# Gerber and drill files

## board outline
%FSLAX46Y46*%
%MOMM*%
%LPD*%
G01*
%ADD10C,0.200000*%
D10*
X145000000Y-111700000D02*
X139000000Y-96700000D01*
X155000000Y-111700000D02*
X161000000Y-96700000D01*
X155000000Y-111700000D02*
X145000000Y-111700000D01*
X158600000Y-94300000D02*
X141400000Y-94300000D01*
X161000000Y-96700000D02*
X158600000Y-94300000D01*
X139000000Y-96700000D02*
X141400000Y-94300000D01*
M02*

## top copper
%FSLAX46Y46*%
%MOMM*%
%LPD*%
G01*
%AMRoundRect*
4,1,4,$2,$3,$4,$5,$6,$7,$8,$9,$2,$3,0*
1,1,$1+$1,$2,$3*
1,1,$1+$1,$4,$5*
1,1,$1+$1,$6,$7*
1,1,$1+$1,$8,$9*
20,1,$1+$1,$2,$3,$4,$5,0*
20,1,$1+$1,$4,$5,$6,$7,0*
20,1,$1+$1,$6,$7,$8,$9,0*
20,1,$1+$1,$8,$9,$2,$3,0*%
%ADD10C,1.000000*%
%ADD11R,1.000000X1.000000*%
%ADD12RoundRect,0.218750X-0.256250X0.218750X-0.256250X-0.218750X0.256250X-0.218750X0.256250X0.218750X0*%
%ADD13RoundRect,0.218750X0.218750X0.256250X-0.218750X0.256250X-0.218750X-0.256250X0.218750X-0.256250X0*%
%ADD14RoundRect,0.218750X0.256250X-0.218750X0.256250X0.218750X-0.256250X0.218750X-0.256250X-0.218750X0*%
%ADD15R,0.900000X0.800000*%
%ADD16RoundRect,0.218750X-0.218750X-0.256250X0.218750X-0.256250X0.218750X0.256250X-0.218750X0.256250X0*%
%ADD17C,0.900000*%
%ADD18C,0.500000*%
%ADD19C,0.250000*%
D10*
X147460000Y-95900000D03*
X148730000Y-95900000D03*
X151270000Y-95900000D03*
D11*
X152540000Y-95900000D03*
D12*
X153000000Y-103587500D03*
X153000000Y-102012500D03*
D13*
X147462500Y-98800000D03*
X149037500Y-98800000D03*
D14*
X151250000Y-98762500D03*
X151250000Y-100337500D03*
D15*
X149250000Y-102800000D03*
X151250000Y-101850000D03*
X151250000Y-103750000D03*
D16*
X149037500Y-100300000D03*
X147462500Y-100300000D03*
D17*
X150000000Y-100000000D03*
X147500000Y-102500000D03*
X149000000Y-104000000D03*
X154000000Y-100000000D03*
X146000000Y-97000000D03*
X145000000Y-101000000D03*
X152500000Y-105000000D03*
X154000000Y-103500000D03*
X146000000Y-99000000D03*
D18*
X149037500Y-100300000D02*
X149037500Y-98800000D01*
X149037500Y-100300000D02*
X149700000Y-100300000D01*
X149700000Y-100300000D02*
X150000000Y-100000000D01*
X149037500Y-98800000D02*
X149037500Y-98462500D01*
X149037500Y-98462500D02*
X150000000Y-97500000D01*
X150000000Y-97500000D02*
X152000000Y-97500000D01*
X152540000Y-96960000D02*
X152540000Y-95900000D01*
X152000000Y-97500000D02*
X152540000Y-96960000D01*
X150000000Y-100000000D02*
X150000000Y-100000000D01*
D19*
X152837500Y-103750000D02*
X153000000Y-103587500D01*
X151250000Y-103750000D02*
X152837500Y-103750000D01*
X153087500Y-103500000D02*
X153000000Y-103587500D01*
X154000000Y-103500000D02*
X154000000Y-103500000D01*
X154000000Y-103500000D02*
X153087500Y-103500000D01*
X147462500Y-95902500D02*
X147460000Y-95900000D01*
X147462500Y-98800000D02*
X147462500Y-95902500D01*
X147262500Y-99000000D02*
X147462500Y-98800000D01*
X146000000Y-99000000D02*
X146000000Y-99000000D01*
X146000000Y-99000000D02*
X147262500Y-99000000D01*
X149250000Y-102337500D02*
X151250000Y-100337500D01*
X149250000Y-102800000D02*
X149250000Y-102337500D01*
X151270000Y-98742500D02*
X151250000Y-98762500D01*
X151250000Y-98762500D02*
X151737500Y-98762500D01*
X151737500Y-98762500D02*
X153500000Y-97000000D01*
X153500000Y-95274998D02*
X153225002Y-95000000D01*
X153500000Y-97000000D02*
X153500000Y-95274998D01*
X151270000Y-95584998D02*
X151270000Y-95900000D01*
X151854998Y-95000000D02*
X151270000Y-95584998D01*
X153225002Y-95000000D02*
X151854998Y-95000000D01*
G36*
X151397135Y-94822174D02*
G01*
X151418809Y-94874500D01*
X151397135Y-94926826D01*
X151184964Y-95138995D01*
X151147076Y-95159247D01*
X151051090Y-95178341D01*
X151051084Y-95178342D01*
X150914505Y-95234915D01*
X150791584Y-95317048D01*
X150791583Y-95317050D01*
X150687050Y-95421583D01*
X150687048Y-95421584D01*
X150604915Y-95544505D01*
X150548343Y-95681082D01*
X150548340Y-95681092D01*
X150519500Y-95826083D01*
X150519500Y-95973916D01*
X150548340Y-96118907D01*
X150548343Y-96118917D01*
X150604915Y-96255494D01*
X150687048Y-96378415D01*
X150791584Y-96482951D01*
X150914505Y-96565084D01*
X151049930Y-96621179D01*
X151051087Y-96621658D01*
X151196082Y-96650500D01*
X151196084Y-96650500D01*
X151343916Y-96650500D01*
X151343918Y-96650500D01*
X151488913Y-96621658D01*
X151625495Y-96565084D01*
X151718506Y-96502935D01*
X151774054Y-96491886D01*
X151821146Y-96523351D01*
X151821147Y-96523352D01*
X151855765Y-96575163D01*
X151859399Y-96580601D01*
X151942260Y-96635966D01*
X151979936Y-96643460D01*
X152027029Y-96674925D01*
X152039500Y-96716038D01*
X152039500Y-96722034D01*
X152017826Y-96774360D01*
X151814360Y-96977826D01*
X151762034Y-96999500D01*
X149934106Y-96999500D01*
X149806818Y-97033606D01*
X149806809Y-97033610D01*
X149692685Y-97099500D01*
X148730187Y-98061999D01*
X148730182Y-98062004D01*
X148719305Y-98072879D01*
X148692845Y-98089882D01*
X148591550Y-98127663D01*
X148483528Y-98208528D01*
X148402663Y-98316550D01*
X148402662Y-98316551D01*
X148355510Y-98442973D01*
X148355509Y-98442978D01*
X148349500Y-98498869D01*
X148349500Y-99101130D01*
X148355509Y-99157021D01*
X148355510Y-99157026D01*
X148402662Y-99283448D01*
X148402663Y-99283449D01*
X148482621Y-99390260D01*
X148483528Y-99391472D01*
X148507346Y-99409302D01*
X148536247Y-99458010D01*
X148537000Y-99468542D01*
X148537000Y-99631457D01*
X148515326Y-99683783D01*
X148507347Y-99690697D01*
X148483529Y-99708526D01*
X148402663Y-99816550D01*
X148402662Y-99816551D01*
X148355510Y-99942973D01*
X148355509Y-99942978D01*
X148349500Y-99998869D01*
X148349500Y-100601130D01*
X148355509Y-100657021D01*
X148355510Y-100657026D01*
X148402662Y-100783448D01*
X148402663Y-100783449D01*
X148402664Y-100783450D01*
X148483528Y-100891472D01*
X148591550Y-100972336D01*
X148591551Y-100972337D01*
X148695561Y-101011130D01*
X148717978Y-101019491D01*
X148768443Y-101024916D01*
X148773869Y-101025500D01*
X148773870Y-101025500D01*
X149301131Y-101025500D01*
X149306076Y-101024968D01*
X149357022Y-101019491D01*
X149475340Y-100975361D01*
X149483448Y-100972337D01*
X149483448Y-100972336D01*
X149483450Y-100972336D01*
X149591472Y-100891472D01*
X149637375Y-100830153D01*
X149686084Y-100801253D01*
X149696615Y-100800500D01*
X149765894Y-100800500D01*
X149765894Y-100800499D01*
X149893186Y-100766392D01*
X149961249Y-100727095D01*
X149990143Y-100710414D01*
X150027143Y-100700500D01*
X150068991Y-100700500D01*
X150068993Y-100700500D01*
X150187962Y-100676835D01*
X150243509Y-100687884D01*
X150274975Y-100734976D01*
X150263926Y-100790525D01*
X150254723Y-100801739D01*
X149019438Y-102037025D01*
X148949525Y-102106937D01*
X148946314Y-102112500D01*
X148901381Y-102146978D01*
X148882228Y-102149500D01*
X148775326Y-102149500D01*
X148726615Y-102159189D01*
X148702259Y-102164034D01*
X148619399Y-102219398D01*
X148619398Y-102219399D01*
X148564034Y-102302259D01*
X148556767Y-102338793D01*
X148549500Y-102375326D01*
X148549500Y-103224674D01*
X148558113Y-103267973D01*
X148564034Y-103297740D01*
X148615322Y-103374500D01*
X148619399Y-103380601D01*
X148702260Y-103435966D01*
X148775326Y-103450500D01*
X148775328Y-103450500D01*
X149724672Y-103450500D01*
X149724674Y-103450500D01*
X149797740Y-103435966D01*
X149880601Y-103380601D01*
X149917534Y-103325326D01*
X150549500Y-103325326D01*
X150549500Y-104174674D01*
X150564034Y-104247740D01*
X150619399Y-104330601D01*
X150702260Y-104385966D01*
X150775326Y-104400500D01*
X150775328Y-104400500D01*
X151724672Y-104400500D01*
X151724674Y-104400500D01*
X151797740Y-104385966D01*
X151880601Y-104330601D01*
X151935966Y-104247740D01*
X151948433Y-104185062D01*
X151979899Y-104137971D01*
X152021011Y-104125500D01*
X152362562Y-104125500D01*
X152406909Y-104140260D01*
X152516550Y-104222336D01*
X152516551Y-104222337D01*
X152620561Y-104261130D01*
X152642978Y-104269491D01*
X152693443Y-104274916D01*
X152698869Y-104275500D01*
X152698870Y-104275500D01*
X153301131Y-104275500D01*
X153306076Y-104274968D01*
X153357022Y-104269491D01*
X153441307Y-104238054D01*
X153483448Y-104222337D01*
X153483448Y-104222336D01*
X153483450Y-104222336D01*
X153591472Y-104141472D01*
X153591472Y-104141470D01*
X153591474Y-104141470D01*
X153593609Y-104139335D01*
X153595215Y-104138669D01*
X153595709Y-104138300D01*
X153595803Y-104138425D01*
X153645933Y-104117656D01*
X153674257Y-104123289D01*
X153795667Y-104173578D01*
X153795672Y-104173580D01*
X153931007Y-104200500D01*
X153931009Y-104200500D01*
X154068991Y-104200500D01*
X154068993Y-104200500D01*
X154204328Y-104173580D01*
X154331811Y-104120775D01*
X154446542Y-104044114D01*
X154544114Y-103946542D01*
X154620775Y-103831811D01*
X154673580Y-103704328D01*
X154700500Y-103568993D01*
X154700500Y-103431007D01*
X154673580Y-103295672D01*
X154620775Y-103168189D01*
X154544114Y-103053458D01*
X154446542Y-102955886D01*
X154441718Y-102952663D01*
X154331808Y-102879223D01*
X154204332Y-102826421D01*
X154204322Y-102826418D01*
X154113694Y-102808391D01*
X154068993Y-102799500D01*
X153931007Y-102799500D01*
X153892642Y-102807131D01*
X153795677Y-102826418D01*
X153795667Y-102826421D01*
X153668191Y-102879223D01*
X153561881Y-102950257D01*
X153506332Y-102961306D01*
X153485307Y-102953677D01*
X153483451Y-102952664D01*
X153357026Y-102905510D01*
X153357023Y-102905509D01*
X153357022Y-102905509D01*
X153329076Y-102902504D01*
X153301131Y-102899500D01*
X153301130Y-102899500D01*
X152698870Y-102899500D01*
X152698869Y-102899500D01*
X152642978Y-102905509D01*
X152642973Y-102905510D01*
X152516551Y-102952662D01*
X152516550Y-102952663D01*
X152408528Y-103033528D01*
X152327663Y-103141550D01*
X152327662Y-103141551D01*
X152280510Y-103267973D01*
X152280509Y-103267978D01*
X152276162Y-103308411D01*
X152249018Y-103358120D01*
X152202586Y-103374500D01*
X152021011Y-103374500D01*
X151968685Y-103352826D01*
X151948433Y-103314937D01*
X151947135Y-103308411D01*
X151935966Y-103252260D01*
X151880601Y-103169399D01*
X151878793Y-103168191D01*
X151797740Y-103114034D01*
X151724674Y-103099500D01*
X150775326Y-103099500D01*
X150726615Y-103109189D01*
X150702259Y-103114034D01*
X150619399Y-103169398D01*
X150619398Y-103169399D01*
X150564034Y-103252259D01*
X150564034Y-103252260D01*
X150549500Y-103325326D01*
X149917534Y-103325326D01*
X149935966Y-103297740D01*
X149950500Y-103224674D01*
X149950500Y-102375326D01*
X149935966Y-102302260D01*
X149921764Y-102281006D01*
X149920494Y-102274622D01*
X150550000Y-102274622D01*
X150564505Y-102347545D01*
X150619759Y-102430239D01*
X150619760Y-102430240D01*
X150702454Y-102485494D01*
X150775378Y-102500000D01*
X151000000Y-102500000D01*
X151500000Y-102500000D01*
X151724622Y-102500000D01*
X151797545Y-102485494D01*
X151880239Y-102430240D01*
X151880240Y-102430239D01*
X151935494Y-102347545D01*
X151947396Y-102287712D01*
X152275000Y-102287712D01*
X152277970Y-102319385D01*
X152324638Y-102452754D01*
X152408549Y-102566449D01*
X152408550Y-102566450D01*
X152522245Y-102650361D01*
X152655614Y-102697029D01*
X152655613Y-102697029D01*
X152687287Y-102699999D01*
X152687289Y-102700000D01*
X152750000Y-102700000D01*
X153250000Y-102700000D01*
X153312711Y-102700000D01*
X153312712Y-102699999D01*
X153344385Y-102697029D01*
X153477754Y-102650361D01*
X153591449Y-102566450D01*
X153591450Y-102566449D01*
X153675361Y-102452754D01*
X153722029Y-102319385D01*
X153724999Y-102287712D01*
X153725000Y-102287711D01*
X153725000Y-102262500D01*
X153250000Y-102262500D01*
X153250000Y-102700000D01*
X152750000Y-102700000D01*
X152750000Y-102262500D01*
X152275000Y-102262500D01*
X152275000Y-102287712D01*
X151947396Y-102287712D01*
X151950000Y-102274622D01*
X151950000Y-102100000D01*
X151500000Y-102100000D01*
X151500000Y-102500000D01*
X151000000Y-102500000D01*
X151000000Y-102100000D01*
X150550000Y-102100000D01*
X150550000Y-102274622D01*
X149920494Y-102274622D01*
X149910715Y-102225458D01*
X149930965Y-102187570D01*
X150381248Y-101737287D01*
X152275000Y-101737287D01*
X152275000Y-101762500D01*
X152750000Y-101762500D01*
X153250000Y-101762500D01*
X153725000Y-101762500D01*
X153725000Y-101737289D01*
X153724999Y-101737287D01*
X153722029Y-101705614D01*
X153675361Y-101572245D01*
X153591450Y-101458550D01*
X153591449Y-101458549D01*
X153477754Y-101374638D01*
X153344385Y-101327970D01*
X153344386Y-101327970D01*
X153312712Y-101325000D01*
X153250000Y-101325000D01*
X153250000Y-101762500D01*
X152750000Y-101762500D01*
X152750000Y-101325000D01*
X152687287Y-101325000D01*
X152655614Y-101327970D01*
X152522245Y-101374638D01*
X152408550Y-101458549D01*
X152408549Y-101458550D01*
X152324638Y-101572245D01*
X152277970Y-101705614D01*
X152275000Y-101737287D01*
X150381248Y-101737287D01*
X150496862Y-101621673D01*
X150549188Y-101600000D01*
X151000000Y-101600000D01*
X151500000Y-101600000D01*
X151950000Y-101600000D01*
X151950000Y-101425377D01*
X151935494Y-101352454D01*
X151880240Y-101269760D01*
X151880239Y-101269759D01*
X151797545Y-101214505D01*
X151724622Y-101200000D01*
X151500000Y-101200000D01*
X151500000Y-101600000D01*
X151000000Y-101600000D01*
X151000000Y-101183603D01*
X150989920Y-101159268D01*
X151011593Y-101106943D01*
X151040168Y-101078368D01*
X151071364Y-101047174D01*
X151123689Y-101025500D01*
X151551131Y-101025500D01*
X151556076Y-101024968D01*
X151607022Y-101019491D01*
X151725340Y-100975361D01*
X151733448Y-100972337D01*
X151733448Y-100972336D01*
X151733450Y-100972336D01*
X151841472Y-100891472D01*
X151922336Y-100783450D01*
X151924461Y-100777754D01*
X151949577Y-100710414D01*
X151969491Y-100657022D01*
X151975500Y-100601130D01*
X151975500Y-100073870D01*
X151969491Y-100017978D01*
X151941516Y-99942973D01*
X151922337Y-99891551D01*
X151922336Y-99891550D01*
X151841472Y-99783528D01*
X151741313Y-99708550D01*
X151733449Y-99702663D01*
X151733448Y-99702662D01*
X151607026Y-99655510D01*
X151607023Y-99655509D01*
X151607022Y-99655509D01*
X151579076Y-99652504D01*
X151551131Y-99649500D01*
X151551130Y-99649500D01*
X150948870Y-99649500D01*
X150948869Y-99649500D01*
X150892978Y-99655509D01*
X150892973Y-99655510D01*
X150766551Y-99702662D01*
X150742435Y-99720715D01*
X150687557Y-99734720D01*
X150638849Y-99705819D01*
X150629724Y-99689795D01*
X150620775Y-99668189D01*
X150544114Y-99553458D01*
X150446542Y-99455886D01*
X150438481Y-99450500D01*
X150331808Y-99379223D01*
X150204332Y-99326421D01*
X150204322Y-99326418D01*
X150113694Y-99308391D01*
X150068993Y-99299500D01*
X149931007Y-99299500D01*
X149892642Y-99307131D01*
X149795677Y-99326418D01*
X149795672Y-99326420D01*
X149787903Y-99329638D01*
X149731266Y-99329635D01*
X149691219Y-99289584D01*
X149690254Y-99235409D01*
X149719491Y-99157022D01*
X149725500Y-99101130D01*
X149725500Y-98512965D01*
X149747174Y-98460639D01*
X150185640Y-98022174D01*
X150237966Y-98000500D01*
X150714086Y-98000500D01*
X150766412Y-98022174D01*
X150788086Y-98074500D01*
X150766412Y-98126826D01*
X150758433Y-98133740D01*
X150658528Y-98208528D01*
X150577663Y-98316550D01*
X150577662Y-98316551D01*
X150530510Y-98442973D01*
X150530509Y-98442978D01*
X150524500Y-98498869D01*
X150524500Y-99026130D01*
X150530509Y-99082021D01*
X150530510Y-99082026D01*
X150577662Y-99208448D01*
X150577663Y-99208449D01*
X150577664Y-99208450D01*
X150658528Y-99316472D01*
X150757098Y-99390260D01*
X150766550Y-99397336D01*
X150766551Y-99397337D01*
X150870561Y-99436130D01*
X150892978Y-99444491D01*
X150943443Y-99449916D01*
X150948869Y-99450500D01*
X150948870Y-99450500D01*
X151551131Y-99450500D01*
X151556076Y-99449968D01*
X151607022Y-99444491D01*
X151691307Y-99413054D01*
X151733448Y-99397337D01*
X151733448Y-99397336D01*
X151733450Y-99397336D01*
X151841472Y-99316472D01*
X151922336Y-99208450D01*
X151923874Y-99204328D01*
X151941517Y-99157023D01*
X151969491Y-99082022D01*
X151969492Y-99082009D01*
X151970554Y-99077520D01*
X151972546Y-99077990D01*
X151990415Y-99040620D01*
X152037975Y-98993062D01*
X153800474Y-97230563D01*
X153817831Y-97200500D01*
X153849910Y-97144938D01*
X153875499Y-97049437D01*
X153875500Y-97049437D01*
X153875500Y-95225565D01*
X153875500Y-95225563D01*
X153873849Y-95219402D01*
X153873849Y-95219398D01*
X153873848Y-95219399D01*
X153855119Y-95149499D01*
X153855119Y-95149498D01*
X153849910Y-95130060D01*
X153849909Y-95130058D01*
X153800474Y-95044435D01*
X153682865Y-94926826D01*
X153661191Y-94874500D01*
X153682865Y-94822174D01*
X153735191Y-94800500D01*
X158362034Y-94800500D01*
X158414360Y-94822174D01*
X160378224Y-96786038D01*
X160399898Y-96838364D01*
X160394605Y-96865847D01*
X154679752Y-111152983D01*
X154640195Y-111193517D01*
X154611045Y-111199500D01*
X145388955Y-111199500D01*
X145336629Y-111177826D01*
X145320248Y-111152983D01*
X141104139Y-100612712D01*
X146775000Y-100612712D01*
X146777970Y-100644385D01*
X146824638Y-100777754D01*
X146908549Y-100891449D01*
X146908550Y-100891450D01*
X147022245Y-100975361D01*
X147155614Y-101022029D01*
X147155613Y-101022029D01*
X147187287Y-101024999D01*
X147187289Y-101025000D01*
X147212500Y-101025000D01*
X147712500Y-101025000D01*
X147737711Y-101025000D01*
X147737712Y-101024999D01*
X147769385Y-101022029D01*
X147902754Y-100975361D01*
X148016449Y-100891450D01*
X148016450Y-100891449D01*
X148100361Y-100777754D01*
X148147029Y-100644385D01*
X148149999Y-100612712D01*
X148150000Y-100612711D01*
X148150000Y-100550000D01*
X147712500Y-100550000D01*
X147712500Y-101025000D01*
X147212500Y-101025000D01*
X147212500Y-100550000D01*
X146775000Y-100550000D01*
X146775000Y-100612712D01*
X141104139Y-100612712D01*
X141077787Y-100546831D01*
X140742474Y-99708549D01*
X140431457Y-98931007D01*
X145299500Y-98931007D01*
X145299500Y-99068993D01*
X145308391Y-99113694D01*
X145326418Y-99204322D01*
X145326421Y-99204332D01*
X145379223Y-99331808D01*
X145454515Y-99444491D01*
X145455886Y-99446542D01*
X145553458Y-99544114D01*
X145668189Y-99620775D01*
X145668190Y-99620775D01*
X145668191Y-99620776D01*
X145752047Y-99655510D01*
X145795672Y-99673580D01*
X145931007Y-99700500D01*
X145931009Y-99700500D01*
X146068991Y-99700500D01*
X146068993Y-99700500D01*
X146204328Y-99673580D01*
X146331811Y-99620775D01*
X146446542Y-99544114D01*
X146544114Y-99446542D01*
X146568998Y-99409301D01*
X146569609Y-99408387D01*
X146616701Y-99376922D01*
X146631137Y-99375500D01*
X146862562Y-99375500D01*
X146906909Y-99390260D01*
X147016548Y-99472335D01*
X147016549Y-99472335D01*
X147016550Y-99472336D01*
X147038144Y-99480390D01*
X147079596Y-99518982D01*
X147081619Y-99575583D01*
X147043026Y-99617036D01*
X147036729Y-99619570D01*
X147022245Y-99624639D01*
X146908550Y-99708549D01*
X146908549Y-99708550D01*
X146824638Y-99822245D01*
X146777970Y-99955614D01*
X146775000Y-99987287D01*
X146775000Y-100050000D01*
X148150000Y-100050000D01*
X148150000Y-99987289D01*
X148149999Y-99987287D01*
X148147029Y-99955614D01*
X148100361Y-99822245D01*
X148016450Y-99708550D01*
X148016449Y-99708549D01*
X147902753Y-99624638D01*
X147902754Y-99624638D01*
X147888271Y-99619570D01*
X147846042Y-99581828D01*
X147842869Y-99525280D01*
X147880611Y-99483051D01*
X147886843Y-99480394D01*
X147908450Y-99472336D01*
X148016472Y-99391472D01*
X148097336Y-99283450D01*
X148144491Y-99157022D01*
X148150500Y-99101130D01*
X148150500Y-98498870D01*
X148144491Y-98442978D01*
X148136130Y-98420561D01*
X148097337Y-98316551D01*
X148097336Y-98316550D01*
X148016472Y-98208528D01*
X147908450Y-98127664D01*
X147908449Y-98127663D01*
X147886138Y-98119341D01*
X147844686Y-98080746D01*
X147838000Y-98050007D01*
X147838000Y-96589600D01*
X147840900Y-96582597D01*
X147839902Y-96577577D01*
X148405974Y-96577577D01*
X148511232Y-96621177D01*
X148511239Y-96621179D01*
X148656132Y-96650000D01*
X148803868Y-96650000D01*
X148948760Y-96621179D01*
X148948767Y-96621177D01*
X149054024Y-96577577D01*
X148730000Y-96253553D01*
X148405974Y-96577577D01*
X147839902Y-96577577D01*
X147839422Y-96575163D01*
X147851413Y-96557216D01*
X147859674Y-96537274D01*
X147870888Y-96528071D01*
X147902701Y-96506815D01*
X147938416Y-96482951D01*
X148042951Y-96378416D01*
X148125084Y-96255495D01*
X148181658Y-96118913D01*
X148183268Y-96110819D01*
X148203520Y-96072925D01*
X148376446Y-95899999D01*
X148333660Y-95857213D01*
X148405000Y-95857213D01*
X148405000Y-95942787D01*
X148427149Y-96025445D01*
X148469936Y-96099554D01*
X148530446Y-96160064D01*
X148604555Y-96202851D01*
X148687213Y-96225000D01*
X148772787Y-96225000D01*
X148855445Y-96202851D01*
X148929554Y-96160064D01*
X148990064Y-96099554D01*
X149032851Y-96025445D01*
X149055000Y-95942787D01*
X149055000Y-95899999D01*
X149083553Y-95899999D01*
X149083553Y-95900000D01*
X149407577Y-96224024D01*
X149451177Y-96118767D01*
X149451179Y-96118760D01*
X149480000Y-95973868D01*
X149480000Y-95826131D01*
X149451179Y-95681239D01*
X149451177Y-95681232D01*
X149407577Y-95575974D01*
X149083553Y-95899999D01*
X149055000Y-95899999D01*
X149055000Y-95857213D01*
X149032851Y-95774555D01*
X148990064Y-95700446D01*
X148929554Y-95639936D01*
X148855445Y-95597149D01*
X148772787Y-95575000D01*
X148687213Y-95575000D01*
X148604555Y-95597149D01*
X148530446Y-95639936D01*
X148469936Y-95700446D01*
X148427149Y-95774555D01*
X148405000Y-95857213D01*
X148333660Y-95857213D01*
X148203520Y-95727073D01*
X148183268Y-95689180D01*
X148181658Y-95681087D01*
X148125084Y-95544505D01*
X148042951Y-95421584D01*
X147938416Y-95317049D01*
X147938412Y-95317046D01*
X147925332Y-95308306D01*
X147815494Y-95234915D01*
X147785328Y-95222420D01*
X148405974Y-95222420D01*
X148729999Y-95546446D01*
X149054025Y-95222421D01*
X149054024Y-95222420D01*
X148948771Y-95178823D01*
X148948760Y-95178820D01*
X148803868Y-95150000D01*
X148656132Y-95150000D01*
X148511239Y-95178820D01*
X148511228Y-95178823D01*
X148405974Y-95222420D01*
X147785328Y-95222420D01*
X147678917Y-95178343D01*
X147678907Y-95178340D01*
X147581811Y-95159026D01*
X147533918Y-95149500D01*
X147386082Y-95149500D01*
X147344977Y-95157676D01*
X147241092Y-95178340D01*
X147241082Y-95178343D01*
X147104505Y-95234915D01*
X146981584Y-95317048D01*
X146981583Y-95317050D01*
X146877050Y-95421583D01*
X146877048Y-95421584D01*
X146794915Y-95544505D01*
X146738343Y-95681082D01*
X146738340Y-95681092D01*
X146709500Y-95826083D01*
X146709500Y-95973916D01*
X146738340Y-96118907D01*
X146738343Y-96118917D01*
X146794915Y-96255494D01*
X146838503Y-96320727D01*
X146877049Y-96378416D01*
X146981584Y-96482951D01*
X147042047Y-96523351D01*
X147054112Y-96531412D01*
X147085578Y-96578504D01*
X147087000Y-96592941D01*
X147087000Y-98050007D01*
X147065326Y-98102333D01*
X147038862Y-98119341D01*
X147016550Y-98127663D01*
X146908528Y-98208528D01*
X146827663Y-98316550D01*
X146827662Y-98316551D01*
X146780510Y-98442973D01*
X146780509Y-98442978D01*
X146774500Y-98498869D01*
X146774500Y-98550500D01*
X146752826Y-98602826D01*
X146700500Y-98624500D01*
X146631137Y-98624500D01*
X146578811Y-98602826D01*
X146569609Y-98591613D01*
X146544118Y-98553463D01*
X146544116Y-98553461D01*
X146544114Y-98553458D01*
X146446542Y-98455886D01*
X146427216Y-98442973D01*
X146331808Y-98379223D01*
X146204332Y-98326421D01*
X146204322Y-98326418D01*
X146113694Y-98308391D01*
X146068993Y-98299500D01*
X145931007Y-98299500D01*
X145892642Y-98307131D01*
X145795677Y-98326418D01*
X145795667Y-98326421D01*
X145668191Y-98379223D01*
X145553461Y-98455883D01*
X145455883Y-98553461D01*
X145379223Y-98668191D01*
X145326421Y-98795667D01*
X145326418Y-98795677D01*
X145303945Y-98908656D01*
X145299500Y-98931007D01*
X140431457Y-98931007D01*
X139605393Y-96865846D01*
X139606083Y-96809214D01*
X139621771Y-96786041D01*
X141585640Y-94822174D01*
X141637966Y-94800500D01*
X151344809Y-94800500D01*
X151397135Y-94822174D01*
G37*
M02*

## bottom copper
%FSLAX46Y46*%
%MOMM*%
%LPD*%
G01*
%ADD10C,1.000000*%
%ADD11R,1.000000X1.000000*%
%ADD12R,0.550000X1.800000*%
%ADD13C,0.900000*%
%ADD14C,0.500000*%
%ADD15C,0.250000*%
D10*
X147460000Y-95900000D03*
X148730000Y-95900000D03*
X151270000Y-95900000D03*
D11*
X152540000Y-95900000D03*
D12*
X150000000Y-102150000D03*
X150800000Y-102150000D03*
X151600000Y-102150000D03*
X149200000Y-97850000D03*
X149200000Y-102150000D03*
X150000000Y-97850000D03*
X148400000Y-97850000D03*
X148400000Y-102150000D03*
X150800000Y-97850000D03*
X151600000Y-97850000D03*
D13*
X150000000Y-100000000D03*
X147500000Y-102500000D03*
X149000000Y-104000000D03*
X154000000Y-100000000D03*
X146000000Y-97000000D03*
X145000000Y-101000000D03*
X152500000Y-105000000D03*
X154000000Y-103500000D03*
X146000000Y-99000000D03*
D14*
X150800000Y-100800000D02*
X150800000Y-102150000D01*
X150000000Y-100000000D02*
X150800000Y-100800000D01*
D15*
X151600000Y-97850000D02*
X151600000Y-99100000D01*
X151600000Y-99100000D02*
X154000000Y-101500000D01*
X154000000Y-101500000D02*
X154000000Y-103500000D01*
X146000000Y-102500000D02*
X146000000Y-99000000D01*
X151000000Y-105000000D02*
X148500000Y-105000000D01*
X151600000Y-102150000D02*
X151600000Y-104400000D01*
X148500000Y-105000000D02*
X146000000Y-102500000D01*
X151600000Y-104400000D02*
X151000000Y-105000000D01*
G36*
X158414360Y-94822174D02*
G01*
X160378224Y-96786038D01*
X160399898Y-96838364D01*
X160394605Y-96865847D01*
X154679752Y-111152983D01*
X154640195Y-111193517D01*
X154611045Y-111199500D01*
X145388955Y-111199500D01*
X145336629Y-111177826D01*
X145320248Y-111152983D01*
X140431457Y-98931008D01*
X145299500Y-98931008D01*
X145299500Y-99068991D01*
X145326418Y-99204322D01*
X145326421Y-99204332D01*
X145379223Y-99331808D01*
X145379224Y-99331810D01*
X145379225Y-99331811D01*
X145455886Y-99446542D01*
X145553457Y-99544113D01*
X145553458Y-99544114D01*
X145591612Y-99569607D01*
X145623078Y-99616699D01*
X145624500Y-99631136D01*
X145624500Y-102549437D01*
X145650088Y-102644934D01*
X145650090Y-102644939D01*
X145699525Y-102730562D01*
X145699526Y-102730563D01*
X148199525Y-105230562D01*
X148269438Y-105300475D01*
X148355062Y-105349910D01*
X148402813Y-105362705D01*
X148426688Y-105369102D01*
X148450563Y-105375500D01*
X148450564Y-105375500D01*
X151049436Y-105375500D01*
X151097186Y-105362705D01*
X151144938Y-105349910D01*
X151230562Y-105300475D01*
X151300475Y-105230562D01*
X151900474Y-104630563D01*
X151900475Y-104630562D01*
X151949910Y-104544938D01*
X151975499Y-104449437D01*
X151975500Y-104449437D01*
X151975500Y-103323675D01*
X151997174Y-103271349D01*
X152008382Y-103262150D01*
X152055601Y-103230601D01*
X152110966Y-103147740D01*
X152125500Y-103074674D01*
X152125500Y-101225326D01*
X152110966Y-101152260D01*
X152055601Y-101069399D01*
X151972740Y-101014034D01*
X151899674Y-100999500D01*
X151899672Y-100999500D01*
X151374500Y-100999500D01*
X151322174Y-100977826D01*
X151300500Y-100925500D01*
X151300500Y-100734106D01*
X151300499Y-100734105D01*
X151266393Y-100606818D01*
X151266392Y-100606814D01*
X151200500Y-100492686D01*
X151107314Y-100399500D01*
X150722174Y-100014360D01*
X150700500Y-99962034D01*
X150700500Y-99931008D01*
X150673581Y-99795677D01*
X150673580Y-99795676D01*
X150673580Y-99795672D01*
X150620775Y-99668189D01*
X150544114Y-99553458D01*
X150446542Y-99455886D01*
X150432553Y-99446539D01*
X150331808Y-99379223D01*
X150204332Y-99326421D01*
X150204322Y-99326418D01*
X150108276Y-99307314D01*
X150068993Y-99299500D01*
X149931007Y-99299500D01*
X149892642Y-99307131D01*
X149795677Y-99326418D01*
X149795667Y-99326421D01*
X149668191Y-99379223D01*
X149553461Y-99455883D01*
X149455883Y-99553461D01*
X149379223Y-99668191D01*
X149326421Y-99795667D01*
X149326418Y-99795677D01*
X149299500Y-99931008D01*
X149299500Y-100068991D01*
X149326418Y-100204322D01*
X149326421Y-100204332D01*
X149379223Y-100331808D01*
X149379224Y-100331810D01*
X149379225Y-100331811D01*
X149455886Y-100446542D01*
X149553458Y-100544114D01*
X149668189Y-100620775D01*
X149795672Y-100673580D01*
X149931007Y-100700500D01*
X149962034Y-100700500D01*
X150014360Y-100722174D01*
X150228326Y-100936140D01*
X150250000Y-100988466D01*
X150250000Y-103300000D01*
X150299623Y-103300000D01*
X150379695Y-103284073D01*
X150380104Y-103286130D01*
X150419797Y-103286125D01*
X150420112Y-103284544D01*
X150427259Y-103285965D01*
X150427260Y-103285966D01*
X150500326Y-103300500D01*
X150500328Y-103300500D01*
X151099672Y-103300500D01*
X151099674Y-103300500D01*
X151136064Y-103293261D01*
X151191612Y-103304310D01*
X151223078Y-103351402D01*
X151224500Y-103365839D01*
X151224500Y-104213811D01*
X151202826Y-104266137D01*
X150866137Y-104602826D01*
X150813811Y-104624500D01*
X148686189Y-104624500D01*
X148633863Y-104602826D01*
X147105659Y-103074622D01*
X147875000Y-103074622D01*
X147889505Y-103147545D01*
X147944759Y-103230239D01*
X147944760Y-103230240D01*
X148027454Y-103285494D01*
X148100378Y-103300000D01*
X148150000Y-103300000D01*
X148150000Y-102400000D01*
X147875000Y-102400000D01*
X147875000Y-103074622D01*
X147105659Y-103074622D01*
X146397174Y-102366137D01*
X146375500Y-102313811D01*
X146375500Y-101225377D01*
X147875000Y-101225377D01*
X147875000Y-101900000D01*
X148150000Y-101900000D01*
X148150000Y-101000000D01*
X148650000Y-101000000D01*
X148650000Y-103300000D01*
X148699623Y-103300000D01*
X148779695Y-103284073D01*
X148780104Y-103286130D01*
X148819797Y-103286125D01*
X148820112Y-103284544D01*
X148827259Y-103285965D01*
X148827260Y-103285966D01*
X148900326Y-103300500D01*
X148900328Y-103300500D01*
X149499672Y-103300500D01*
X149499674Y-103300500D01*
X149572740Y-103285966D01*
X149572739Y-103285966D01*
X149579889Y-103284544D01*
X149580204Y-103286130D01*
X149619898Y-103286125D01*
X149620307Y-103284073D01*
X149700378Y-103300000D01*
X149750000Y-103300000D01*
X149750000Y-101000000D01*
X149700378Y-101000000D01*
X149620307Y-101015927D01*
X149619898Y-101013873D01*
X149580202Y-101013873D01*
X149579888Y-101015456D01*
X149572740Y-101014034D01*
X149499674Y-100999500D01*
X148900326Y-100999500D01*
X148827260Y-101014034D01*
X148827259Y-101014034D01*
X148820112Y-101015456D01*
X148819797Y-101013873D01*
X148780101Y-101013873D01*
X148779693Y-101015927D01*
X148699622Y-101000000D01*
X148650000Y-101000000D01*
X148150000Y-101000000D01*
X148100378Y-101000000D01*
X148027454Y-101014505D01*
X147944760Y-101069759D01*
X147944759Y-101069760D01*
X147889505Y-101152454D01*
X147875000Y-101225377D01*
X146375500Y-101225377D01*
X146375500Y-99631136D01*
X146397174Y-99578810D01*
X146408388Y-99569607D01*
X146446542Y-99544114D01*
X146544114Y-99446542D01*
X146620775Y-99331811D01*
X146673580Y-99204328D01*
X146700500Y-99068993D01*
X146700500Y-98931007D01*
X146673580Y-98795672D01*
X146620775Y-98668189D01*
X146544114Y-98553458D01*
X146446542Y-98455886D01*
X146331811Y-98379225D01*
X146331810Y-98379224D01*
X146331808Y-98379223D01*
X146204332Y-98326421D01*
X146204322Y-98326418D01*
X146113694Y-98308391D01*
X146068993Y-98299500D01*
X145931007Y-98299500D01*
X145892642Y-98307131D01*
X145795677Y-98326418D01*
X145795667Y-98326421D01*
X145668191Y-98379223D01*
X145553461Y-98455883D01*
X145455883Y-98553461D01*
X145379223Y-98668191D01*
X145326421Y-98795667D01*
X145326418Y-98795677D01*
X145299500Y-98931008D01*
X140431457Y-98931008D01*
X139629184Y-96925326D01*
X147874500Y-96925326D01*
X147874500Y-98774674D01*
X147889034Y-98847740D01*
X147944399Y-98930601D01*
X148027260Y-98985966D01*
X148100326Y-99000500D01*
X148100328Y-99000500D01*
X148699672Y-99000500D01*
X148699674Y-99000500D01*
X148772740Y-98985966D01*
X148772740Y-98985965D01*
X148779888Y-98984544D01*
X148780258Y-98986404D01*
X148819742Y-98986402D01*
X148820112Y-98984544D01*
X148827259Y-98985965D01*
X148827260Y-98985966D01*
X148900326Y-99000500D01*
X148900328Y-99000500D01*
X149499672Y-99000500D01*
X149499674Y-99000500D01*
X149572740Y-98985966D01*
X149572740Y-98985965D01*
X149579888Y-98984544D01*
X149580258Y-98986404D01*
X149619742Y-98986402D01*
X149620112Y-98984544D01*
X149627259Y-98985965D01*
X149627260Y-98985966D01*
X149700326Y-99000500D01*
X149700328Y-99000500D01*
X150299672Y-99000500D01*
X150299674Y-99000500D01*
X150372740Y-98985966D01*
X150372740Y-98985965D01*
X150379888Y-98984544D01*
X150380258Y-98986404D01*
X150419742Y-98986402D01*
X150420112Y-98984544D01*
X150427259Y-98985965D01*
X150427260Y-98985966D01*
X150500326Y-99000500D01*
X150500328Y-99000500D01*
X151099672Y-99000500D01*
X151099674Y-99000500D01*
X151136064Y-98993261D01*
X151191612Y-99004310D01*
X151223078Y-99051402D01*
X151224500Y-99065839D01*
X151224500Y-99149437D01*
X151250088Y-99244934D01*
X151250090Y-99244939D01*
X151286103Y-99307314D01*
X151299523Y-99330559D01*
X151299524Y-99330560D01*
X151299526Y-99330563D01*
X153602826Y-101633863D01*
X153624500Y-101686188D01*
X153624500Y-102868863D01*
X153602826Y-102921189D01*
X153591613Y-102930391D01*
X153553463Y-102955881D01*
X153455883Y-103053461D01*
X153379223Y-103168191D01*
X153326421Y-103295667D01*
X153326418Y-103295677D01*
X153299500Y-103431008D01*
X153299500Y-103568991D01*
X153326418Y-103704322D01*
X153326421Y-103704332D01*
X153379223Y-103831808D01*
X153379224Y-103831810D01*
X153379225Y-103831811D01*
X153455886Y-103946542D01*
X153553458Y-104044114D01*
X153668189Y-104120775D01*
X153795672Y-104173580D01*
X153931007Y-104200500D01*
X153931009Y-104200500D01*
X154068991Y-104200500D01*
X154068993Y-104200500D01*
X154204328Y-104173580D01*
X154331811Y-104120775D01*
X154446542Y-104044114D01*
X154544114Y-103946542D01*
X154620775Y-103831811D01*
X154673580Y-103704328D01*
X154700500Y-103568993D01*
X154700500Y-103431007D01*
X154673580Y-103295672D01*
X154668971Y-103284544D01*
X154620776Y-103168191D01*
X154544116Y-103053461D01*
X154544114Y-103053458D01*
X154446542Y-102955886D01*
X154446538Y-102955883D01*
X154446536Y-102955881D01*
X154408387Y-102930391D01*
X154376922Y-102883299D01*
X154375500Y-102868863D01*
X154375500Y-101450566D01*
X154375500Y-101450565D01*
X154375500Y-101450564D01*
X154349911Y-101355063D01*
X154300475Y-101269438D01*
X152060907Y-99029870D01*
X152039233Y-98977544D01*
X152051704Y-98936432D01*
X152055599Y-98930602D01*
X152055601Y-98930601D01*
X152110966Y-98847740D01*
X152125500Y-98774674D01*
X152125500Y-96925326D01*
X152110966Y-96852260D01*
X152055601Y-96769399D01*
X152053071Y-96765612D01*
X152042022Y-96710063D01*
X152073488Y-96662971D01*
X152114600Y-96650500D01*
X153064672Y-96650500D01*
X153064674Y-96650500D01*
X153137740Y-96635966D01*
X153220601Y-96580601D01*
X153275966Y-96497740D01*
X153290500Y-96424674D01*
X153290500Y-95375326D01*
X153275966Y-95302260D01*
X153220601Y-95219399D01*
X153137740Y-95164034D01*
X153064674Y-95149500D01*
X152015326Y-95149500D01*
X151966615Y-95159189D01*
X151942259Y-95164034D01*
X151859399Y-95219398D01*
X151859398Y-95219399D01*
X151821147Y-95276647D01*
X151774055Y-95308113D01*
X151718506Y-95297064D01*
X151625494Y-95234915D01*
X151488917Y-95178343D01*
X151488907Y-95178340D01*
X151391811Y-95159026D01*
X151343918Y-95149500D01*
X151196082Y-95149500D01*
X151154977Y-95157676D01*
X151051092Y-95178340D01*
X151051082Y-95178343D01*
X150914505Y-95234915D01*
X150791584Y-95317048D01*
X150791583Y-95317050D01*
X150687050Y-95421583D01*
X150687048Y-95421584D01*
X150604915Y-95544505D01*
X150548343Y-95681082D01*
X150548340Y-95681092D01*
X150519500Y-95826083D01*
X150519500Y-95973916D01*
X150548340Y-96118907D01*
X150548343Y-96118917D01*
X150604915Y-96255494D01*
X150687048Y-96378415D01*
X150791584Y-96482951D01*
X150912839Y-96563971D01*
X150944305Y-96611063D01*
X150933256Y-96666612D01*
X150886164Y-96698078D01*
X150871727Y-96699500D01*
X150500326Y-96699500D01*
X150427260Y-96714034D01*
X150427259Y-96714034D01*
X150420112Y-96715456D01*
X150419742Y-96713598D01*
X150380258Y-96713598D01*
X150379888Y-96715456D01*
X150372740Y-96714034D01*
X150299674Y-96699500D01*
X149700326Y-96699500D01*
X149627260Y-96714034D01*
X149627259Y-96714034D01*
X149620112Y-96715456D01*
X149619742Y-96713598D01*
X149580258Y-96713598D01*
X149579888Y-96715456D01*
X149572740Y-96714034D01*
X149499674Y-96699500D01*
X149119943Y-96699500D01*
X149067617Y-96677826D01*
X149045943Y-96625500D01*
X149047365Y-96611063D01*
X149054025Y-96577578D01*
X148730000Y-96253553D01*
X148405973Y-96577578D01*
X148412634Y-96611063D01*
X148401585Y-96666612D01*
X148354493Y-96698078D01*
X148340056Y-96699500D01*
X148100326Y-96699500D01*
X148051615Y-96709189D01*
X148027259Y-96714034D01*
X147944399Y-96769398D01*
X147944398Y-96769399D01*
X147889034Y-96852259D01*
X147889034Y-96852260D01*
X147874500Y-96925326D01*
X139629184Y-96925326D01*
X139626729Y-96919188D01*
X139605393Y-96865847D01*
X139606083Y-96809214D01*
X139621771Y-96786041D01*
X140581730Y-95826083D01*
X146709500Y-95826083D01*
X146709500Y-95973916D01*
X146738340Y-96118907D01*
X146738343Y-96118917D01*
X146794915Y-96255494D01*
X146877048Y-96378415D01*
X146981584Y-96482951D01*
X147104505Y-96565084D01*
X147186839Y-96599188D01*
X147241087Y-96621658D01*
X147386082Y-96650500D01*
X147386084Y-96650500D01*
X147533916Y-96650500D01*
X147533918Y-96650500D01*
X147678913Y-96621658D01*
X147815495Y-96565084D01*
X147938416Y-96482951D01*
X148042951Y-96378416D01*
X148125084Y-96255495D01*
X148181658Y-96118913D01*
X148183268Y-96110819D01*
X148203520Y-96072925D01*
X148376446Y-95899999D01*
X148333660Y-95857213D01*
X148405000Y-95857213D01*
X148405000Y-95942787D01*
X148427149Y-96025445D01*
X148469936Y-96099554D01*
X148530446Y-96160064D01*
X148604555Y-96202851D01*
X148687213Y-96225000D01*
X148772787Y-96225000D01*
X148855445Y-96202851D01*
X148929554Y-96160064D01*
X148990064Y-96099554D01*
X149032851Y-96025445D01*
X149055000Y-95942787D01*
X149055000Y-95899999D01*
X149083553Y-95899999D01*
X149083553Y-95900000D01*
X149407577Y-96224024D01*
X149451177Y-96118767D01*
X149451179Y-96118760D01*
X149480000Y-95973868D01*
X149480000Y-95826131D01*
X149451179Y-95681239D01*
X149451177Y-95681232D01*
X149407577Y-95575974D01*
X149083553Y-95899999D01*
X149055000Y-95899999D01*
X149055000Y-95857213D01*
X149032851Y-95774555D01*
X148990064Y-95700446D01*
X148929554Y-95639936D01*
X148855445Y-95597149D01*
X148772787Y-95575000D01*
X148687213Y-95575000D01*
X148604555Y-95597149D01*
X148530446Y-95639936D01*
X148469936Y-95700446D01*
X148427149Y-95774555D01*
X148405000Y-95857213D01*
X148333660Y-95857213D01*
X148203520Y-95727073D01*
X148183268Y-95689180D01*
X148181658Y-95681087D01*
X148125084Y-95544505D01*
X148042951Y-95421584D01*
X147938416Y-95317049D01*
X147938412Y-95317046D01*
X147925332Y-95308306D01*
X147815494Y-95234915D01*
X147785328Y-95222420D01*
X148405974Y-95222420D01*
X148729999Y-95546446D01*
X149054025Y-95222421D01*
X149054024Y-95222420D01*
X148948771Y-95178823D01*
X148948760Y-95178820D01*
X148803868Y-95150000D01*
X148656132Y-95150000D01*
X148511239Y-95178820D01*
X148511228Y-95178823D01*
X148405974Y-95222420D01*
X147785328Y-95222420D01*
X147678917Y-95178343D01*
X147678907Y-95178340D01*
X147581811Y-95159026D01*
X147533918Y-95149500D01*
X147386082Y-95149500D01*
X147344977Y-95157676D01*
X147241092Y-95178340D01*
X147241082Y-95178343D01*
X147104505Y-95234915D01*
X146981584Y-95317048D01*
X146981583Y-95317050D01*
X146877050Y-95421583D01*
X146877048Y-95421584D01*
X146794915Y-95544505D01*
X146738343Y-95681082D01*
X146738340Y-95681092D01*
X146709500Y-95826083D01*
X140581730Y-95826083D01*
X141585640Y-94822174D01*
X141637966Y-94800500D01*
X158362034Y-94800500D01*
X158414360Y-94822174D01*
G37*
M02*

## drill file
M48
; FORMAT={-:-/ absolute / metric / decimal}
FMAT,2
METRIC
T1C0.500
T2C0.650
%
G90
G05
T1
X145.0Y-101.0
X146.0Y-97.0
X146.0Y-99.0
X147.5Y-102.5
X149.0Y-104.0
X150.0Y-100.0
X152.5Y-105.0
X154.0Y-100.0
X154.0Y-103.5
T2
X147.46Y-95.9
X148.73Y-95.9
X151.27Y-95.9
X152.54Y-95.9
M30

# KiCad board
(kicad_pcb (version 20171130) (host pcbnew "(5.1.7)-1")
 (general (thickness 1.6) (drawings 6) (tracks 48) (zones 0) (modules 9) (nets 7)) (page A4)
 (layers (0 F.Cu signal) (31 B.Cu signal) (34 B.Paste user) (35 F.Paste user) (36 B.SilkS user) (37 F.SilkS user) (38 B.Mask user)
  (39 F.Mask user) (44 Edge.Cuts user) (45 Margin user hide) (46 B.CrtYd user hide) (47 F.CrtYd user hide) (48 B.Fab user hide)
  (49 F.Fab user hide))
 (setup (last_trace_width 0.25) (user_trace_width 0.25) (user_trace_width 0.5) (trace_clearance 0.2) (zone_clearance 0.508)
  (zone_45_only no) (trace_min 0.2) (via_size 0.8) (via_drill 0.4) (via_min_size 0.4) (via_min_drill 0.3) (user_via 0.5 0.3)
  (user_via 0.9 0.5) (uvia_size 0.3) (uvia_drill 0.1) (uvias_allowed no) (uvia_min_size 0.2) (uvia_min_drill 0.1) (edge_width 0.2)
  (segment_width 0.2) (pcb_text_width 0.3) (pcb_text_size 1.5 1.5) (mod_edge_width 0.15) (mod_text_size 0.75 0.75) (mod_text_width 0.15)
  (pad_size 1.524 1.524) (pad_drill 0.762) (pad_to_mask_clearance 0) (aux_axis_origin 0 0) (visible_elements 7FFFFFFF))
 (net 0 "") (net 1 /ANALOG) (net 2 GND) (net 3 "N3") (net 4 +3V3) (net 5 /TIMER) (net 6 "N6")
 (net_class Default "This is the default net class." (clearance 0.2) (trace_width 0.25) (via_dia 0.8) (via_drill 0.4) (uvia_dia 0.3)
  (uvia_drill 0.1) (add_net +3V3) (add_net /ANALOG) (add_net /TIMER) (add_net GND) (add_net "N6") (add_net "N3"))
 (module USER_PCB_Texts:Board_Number (layer B.Cu) (at 145.5 109)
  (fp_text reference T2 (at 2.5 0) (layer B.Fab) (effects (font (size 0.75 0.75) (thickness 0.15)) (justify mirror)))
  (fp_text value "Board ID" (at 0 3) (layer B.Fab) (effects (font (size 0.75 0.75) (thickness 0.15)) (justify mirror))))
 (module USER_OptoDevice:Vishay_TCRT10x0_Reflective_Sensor (layer F.Cu) (at 150 95.9 180)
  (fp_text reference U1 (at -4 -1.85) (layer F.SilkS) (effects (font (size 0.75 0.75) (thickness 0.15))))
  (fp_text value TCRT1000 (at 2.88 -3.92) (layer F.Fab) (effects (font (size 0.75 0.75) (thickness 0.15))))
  (pad 4 thru_hole circle (at 2.54 0 180) (size 1 1) (drill 0.65) (layers *.Cu *.Mask) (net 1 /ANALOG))
  (pad 3 thru_hole circle (at 1.27 0 180) (size 1 1) (drill 0.65) (layers *.Cu *.Mask) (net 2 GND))
  (pad 2 thru_hole circle (at -1.27 0 180) (size 1 1) (drill 0.65) (layers *.Cu *.Mask) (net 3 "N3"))
  (pad 1 thru_hole rect (at -2.54 0 180) (size 1 1) (drill 0.65) (layers *.Cu *.Mask) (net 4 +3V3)))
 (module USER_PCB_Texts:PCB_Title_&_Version (layer F.Cu) (at 158.414999 105.394999)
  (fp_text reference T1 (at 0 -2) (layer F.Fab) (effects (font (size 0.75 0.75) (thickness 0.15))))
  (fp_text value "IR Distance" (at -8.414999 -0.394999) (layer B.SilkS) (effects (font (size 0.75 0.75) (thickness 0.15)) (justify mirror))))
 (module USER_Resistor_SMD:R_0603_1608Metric (layer F.Cu) (at 153 102.8 270)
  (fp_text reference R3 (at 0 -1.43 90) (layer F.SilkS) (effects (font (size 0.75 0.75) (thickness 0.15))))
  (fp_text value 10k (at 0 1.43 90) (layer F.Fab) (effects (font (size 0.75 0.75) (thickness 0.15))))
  (pad 2 smd roundrect (at 0.7875 0 270) (size 0.875 0.95) (layers F.Cu F.Paste F.Mask) (roundrect_rratio 0.25) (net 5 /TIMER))
  (pad 1 smd roundrect (at -0.7875 0 270) (size 0.875 0.95) (layers F.Cu F.Paste F.Mask) (roundrect_rratio 0.25) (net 2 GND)))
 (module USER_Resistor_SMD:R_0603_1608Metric (layer F.Cu) (at 148.25 98.8 180)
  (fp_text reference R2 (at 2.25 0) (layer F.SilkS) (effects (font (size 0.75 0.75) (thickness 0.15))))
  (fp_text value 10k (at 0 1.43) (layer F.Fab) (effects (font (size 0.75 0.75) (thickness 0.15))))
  (pad 2 smd roundrect (at 0.7875 0 180) (size 0.875 0.95) (layers F.Cu F.Paste F.Mask) (roundrect_rratio 0.25) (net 1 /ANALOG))
  (pad 1 smd roundrect (at -0.7875 0 180) (size 0.875 0.95) (layers F.Cu F.Paste F.Mask) (roundrect_rratio 0.25) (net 4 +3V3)))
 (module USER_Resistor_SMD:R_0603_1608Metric (layer F.Cu) (at 151.25 99.55 90)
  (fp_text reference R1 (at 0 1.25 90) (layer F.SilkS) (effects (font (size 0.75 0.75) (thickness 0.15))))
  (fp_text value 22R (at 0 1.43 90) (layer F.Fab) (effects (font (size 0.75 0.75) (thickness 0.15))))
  (pad 2 smd roundrect (at 0.7875 0 90) (size 0.875 0.95) (layers F.Cu F.Paste F.Mask) (roundrect_rratio 0.25) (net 3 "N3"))
  (pad 1 smd roundrect (at -0.7875 0 90) (size 0.875 0.95) (layers F.Cu F.Paste F.Mask) (roundrect_rratio 0.25) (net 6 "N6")))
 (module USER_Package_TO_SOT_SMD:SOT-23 (layer F.Cu) (at 150.25 102.8 180)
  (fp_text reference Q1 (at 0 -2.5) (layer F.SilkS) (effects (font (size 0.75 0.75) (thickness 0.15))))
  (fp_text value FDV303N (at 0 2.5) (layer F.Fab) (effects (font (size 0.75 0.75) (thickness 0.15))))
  (pad 3 smd rect (at 1 0 180) (size 0.9 0.8) (layers F.Cu F.Paste F.Mask) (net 6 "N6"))
  (pad 2 smd rect (at -1 0.95 180) (size 0.9 0.8) (layers F.Cu F.Paste F.Mask) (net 2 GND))
  (pad 1 smd rect (at -1 -0.95 180) (size 0.9 0.8) (layers F.Cu F.Paste F.Mask) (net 5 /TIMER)))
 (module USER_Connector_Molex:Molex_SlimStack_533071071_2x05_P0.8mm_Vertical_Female (layer B.Cu) (at 150 100 180)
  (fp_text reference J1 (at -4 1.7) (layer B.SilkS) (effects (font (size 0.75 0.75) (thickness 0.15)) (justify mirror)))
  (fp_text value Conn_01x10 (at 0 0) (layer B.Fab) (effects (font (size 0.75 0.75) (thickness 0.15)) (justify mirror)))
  (pad 5 smd rect (at 0 -2.15) (size 0.55 1.8) (layers B.Cu B.Paste B.Mask) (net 2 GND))
  (pad 3 smd rect (at -0.8 -2.15) (size 0.55 1.8) (layers B.Cu B.Paste B.Mask) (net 4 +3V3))
  (pad 1 smd rect (at -1.6 -2.15) (size 0.55 1.8) (layers B.Cu B.Paste B.Mask) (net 1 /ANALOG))
  (pad 8 smd rect (at 0.8 2.15) (size 0.55 1.8) (layers B.Cu B.Paste B.Mask))
  (pad 7 smd rect (at 0.8 -2.15) (size 0.55 1.8) (layers B.Cu B.Paste B.Mask))
  (pad 6 smd rect (at 0 2.15) (size 0.55 1.8) (layers B.Cu B.Paste B.Mask))
  (pad 10 smd rect (at 1.6 2.15) (size 0.55 1.8) (layers B.Cu B.Paste B.Mask))
  (pad 9 smd rect (at 1.6 -2.15) (size 0.55 1.8) (layers B.Cu B.Paste B.Mask) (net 2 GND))
  (pad 4 smd rect (at -0.8 2.15) (size 0.55 1.8) (layers B.Cu B.Paste B.Mask))
  (pad 2 smd rect (at -1.6 2.15) (size 0.55 1.8) (layers B.Cu B.Paste B.Mask) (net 5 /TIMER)))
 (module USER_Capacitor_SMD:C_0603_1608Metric (layer F.Cu) (at 148.25 100.3)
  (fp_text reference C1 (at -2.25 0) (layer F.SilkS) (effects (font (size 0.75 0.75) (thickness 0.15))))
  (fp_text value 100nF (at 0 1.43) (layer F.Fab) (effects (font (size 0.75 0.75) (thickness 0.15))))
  (pad 2 smd roundrect (at 0.7875 0) (size 0.875 0.95) (layers F.Cu F.Paste F.Mask) (roundrect_rratio 0.25) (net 4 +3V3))
  (pad 1 smd roundrect (at -0.7875 0) (size 0.875 0.95) (layers F.Cu F.Paste F.Mask) (roundrect_rratio 0.25) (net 2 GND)))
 (gr_line (start 145 111.7) (end 139 96.7) (layer Edge.Cuts) (width 0.2))
 (gr_line (start 155 111.7) (end 161 96.7) (layer Edge.Cuts) (width 0.2))
 (gr_line (start 155 111.7) (end 145 111.7) (layer Edge.Cuts) (width 0.2))
 (gr_line (start 158.6 94.3) (end 141.4 94.3) (layer Edge.Cuts) (width 0.2))
 (gr_line (start 161 96.7) (end 158.6 94.3) (layer Edge.Cuts) (width 0.2))
 (gr_line (start 139 96.7) (end 141.4 94.3) (layer Edge.Cuts) (width 0.2))
 (segment (start 149.0375 100.3) (end 149.0375 98.8) (width 0.5) (layer F.Cu) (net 4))
 (segment (start 149.0375 100.3) (end 149.7 100.3) (width 0.5) (layer F.Cu) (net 4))
 (segment (start 149.7 100.3) (end 150 100) (width 0.5) (layer F.Cu) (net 4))
 (segment (start 150.8 100.8) (end 150.8 102.15) (width 0.5) (layer B.Cu) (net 4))
 (segment (start 150 100) (end 150.8 100.8) (width 0.5) (layer B.Cu) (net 4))
 (segment (start 149.0375 98.8) (end 149.0375 98.4625) (width 0.5) (layer F.Cu) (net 4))
 (segment (start 149.0375 98.4625) (end 150 97.5) (width 0.5) (layer F.Cu) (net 4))
 (segment (start 150 97.5) (end 152 97.5) (width 0.5) (layer F.Cu) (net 4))
 (segment (start 152.54 96.96) (end 152.54 95.9) (width 0.5) (layer F.Cu) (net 4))
 (segment (start 152 97.5) (end 152.54 96.96) (width 0.5) (layer F.Cu) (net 4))
 (segment (start 150 100) (end 150 100) (width 0.5) (layer F.Cu) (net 4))
 (via (at 150 100) (size 0.9) (drill 0.5) (layers F.Cu B.Cu) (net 4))
 (via (at 147.5 102.5) (size 0.9) (drill 0.5) (layers F.Cu B.Cu) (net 2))
 (via (at 149 104) (size 0.9) (drill 0.5) (layers F.Cu B.Cu) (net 2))
 (via (at 154 100) (size 0.9) (drill 0.5) (layers F.Cu B.Cu) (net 2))
 (via (at 146 97) (size 0.9) (drill 0.5) (layers F.Cu B.Cu) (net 2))
 (via (at 145 101) (size 0.9) (drill 0.5) (layers F.Cu B.Cu) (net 2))
 (via (at 152.5 105) (size 0.9) (drill 0.5) (layers F.Cu B.Cu) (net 2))
 (segment (start 152.8375 103.75) (end 153 103.5875) (width 0.25) (layer F.Cu) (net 5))
 (segment (start 151.25 103.75) (end 152.8375 103.75) (width 0.25) (layer F.Cu) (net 5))
 (segment (start 151.6 97.85) (end 151.6 99.1) (width 0.25) (layer B.Cu) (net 5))
 (segment (start 151.6 99.1) (end 154 101.5) (width 0.25) (layer B.Cu) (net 5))
 (segment (start 154 101.5) (end 154 103.5) (width 0.25) (layer B.Cu) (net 5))
 (segment (start 153.0875 103.5) (end 153 103.5875) (width 0.25) (layer F.Cu) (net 5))
 (segment (start 154 103.5) (end 154 103.5) (width 0.25) (layer F.Cu) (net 5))
 (segment (start 154 103.5) (end 153.0875 103.5) (width 0.25) (layer F.Cu) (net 5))
 (via (at 154 103.5) (size 0.9) (drill 0.5) (layers F.Cu B.Cu) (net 5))
 (segment (start 147.4625 95.9025) (end 147.46 95.9) (width 0.25) (layer F.Cu) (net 1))
 (segment (start 147.4625 98.8) (end 147.4625 95.9025) (width 0.25) (layer F.Cu) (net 1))
 (segment (start 147.2625 99) (end 147.4625 98.8) (width 0.25) (layer F.Cu) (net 1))
 (segment (start 146 99) (end 146 99) (width 0.25) (layer F.Cu) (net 1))
 (segment (start 146 99) (end 147.2625 99) (width 0.25) (layer F.Cu) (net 1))
 (via (at 146 99) (size 0.9) (drill 0.5) (layers F.Cu B.Cu) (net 1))
 (segment (start 146 102.5) (end 146 99) (width 0.25) (layer B.Cu) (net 1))
 (segment (start 151 105) (end 148.5 105) (width 0.25) (layer B.Cu) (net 1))
 (segment (start 151.6 102.15) (end 151.6 104.4) (width 0.25) (layer B.Cu) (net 1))
 (segment (start 148.5 105) (end 146 102.5) (width 0.25) (layer B.Cu) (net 1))
 (segment (start 151.6 104.4) (end 151 105) (width 0.25) (layer B.Cu) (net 1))
 (segment (start 149.25 102.3375) (end 151.25 100.3375) (width 0.25) (layer F.Cu) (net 6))
 (segment (start 149.25 102.8) (end 149.25 102.3375) (width 0.25) (layer F.Cu) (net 6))
 (segment (start 151.27 98.7425) (end 151.25 98.7625) (width 0.25) (layer F.Cu) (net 3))
 (segment (start 151.25 98.7625) (end 151.7375 98.7625) (width 0.25) (layer F.Cu) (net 3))
 (segment (start 151.7375 98.7625) (end 153.5 97) (width 0.25) (layer F.Cu) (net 3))
 (segment (start 153.5 95.274998) (end 153.225002 95) (width 0.25) (layer F.Cu) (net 3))
 (segment (start 153.5 97) (end 153.5 95.274998) (width 0.25) (layer F.Cu) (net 3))
 (segment (start 151.27 95.584998) (end 151.27 95.9) (width 0.25) (layer F.Cu) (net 3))
 (segment (start 151.854998 95) (end 151.27 95.584998) (width 0.25) (layer F.Cu) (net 3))
 (segment (start 153.225002 95) (end 151.854998 95) (width 0.25) (layer F.Cu) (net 3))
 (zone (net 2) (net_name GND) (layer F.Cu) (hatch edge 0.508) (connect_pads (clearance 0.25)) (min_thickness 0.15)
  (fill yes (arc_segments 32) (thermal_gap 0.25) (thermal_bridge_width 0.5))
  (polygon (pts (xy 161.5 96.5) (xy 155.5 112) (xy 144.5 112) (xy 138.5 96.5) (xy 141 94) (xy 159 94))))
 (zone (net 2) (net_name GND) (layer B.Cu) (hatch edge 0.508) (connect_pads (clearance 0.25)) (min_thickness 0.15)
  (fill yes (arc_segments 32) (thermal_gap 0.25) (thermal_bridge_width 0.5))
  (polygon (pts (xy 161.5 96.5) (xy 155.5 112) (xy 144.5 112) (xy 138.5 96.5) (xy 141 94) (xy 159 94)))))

